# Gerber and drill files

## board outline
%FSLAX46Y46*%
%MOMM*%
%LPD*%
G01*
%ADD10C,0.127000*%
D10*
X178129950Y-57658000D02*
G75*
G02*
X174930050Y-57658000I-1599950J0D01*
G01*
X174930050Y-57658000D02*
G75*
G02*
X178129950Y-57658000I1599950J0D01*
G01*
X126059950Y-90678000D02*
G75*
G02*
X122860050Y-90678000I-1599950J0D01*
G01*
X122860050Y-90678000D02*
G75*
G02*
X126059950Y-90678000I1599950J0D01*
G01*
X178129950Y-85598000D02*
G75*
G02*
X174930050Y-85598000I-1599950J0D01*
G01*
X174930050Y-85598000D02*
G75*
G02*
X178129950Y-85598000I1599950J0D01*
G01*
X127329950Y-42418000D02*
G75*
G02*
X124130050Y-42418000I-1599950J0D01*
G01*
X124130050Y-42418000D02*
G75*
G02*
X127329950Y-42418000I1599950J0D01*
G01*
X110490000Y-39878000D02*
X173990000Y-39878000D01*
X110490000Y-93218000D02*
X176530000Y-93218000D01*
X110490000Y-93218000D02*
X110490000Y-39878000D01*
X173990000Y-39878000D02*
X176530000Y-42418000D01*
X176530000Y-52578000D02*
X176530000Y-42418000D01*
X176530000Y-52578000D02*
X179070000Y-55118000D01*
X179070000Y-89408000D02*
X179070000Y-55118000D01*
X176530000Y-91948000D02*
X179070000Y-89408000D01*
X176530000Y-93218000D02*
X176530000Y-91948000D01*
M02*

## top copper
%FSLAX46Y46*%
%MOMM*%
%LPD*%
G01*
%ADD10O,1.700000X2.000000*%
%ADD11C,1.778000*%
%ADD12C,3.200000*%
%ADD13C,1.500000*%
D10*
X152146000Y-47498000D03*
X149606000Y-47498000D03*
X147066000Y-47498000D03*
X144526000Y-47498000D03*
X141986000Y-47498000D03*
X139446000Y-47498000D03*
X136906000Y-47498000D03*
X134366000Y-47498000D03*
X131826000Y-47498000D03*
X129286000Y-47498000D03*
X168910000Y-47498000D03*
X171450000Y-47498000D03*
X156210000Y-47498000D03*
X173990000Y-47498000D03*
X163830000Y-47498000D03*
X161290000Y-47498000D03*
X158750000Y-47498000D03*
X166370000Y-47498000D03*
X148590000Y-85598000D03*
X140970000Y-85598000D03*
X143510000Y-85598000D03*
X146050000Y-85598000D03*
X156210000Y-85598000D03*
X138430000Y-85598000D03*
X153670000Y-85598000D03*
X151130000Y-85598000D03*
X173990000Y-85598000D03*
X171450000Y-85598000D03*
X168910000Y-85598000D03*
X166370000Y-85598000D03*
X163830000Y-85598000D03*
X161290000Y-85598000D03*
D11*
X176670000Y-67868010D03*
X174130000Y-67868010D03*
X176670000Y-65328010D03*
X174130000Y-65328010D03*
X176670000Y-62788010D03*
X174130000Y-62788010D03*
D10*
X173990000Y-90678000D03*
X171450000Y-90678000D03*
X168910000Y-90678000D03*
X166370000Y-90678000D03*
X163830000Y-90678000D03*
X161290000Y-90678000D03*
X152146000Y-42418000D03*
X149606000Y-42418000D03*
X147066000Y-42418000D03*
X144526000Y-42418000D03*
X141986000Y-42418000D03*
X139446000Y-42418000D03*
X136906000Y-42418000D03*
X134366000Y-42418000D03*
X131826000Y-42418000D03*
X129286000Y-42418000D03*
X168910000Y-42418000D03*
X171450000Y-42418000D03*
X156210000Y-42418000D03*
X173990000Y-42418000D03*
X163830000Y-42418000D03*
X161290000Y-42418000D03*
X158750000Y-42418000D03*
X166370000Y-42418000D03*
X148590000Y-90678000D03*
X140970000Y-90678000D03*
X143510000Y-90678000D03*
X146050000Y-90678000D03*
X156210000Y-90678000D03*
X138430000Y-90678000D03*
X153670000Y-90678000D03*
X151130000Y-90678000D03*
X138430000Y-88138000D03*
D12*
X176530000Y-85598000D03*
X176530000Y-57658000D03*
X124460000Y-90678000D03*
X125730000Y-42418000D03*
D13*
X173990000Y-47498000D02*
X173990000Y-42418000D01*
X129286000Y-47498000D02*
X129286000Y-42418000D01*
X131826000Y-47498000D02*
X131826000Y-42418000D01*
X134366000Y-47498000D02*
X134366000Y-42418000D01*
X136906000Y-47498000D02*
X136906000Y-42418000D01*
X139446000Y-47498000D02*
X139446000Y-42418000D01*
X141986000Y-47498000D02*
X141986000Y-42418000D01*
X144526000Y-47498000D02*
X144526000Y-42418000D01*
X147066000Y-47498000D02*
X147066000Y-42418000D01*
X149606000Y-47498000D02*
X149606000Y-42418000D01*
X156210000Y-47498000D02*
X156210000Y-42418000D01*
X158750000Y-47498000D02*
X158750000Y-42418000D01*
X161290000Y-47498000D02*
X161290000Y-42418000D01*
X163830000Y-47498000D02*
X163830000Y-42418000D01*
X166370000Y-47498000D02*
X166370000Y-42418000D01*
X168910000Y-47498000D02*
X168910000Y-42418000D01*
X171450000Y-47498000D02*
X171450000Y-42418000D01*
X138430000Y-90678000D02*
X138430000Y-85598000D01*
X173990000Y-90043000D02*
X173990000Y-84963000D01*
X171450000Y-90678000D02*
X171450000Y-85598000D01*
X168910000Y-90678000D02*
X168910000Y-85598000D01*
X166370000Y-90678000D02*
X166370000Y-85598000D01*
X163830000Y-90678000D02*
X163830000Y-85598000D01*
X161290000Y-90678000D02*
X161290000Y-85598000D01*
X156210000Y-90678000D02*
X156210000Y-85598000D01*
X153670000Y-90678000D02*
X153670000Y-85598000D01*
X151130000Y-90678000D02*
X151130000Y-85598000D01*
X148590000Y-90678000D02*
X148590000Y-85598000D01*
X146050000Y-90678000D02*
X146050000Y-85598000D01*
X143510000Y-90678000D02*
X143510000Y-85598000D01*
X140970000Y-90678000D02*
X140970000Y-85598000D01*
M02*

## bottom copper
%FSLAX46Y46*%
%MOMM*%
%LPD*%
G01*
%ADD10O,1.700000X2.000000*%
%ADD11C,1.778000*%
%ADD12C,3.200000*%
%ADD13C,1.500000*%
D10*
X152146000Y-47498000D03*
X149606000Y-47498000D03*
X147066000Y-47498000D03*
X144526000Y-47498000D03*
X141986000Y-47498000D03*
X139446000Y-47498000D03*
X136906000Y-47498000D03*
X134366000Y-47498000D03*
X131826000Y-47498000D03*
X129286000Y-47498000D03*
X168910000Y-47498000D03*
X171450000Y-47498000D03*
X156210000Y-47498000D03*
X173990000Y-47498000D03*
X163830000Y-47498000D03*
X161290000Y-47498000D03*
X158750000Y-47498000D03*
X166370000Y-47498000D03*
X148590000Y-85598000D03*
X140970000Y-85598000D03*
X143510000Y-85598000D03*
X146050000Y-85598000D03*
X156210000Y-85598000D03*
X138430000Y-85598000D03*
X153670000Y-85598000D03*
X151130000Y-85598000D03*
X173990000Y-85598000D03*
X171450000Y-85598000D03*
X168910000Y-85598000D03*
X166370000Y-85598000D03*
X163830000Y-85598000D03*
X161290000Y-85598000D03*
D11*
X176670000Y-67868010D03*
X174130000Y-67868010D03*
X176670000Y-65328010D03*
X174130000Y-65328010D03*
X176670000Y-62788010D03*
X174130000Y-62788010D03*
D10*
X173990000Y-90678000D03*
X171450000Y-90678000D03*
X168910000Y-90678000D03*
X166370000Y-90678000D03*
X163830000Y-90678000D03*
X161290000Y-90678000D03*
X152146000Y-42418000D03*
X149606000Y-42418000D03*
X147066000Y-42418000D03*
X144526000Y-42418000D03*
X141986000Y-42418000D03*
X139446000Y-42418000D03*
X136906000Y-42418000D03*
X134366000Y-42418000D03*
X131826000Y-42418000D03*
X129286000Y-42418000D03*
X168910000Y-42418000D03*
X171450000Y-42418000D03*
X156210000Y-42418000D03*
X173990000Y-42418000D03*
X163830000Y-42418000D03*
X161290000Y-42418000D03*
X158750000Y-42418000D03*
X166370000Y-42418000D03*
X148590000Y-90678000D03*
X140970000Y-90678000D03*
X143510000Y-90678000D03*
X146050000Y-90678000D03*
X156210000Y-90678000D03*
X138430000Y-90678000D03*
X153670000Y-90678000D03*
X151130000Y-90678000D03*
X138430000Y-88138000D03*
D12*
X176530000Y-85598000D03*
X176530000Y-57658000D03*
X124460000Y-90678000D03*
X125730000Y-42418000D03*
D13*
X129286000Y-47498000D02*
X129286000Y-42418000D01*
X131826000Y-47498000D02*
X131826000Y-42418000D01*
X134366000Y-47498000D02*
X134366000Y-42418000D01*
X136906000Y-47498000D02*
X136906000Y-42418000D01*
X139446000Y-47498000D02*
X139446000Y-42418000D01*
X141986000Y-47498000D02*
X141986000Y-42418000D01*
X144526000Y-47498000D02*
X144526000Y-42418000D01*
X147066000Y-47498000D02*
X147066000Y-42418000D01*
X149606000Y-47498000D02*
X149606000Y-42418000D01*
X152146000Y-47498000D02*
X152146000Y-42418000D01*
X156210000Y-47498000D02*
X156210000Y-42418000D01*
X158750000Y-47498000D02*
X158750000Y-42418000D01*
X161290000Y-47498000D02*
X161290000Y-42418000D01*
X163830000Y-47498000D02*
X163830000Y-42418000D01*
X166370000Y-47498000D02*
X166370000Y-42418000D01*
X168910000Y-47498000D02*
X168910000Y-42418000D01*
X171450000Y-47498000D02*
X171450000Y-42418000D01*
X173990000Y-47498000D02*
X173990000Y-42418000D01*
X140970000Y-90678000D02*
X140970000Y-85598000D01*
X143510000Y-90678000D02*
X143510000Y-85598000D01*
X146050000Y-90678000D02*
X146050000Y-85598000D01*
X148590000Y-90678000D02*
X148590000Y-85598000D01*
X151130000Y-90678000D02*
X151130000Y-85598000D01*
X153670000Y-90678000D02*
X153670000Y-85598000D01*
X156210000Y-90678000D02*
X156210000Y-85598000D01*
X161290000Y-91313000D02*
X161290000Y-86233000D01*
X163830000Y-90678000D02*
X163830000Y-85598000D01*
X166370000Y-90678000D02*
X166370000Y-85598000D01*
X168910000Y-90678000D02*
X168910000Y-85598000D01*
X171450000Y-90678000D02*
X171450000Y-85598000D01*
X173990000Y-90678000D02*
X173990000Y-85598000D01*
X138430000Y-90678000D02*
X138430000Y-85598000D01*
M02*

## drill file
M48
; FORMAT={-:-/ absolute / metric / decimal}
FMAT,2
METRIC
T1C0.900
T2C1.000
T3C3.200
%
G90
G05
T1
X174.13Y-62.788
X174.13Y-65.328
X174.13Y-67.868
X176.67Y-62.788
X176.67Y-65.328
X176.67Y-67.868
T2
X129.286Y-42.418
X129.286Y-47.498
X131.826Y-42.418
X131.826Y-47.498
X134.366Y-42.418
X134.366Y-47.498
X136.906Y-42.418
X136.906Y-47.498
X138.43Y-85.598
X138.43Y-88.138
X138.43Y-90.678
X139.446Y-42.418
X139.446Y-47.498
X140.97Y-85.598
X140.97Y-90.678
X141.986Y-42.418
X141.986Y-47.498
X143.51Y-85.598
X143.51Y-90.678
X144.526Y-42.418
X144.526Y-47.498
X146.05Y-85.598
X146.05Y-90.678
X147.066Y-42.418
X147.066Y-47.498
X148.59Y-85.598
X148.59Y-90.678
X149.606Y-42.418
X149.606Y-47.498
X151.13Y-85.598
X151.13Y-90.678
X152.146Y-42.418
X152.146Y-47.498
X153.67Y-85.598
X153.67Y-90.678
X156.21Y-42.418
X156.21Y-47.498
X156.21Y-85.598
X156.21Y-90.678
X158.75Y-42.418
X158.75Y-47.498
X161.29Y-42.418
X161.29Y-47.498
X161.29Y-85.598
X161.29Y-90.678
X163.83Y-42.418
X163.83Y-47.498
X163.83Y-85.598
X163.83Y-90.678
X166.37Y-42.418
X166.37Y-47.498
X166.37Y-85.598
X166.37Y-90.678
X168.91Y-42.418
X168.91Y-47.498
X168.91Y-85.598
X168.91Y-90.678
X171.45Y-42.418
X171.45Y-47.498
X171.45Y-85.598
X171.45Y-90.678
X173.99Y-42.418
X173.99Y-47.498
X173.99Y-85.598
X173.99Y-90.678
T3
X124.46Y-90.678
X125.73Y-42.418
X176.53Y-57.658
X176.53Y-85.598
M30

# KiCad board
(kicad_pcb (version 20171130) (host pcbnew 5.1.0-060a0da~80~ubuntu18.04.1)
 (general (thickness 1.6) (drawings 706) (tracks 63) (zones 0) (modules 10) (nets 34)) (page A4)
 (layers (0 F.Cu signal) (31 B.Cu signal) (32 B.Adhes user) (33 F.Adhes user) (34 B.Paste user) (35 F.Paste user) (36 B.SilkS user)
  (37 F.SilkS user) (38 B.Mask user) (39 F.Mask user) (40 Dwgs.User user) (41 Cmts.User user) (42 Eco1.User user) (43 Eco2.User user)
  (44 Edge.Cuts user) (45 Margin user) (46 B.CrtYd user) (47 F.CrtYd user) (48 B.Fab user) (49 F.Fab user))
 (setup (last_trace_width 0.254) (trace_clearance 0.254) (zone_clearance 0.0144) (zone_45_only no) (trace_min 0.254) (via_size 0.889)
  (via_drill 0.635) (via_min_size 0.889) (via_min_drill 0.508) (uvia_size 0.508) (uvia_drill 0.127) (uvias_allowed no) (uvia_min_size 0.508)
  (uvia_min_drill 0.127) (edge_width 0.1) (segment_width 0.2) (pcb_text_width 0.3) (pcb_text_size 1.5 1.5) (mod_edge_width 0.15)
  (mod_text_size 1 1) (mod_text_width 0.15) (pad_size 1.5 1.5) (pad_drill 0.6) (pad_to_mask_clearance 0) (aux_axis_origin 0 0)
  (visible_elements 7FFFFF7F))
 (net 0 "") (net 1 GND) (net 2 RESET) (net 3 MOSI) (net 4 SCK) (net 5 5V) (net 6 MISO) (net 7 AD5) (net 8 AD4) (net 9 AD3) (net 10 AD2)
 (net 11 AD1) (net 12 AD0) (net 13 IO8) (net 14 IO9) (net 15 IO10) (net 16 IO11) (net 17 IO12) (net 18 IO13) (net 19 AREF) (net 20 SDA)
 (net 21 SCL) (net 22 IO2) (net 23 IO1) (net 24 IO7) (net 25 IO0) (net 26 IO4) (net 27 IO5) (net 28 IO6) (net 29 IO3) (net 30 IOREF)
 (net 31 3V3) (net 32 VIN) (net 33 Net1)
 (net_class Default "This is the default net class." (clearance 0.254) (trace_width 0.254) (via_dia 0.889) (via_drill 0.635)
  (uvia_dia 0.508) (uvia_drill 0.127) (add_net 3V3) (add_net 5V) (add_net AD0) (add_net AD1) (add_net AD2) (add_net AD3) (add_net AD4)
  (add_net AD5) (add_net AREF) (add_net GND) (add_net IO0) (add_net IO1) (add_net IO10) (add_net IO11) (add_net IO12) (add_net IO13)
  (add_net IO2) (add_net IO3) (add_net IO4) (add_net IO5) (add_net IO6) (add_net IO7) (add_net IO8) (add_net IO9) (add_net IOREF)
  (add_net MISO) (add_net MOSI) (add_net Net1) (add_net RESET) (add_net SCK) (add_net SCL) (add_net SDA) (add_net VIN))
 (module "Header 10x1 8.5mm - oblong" (layer F.Cu) (at 152.146 47.498)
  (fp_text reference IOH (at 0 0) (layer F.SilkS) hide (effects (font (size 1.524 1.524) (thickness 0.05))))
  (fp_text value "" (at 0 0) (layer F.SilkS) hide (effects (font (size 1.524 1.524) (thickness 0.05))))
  (pad 1 thru_hole oval (at 0 0 180) (size 1.7 2) (drill 1) (layers *.Cu *.Paste *.Mask))
  (pad 2 thru_hole oval (at -2.54 0 180) (size 1.7 2) (drill 1) (layers *.Cu *.Paste *.Mask))
  (pad 3 thru_hole oval (at -5.08 0 180) (size 1.7 2) (drill 1) (layers *.Cu *.Paste *.Mask))
  (pad 4 thru_hole oval (at -7.62 0 180) (size 1.7 2) (drill 1) (layers *.Cu *.Paste *.Mask))
  (pad 5 thru_hole oval (at -10.16 0 180) (size 1.7 2) (drill 1) (layers *.Cu *.Paste *.Mask))
  (pad 6 thru_hole oval (at -12.7 0 180) (size 1.7 2) (drill 1) (layers *.Cu *.Paste *.Mask))
  (pad 7 thru_hole oval (at -15.24 0 180) (size 1.7 2) (drill 1) (layers *.Cu *.Paste *.Mask))
  (pad 8 thru_hole oval (at -17.78 0 180) (size 1.7 2) (drill 1) (layers *.Cu *.Paste *.Mask))
  (pad 9 thru_hole oval (at -20.32 0 180) (size 1.7 2) (drill 1) (layers *.Cu *.Paste *.Mask))
  (pad 10 thru_hole oval (at -22.86 0 180) (size 1.7 2) (drill 1) (layers *.Cu *.Paste *.Mask)))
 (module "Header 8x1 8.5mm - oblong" (layer F.Cu) (at 173.99 47.498)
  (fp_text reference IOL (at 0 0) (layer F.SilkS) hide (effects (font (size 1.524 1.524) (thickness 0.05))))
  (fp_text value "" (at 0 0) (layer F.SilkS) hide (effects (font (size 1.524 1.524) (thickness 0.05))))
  (pad 3 thru_hole oval (at -5.08 0 180) (size 1.7 2) (drill 1) (layers *.Cu *.Paste *.Mask))
  (pad 2 thru_hole oval (at -2.54 0 180) (size 1.7 2) (drill 1) (layers *.Cu *.Paste *.Mask))
  (pad 8 thru_hole oval (at -17.78 0 180) (size 1.7 2) (drill 1) (layers *.Cu *.Paste *.Mask))
  (pad 1 thru_hole oval (at 0 0 180) (size 1.7 2) (drill 1) (layers *.Cu *.Paste *.Mask))
  (pad 5 thru_hole oval (at -10.16 0 180) (size 1.7 2) (drill 1) (layers *.Cu *.Paste *.Mask))
  (pad 6 thru_hole oval (at -12.7 0 180) (size 1.7 2) (drill 1) (layers *.Cu *.Paste *.Mask))
  (pad 7 thru_hole oval (at -15.24 0 180) (size 1.7 2) (drill 1) (layers *.Cu *.Paste *.Mask))
  (pad 4 thru_hole oval (at -7.62 0 180) (size 1.7 2) (drill 1) (layers *.Cu *.Paste *.Mask)))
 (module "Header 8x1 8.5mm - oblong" (layer F.Cu) (at 156.21 85.598)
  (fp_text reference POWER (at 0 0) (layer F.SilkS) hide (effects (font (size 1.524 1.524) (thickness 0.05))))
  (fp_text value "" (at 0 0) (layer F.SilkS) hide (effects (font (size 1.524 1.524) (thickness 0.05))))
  (pad 4 thru_hole oval (at -7.62 0 180) (size 1.7 2) (drill 1) (layers *.Cu *.Paste *.Mask))
  (pad 7 thru_hole oval (at -15.24 0 180) (size 1.7 2) (drill 1) (layers *.Cu *.Paste *.Mask))
  (pad 6 thru_hole oval (at -12.7 0 180) (size 1.7 2) (drill 1) (layers *.Cu *.Paste *.Mask))
  (pad 5 thru_hole oval (at -10.16 0 180) (size 1.7 2) (drill 1) (layers *.Cu *.Paste *.Mask))
  (pad 1 thru_hole oval (at 0 0 180) (size 1.7 2) (drill 1) (layers *.Cu *.Paste *.Mask))
  (pad 8 thru_hole oval (at -17.78 0 180) (size 1.7 2) (drill 1) (layers *.Cu *.Paste *.Mask))
  (pad 2 thru_hole oval (at -2.54 0 180) (size 1.7 2) (drill 1) (layers *.Cu *.Paste *.Mask))
  (pad 3 thru_hole oval (at -5.08 0 180) (size 1.7 2) (drill 1) (layers *.Cu *.Paste *.Mask)))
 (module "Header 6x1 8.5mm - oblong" (layer F.Cu) (at 161.29 85.598)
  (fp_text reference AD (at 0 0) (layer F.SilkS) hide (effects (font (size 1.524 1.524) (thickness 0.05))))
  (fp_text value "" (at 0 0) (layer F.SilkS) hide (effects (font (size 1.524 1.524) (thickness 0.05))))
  (pad 6 thru_hole oval (at 12.7 0) (size 1.7 2) (drill 1) (layers *.Cu *.Paste *.Mask))
  (pad 5 thru_hole oval (at 10.16 0) (size 1.7 2) (drill 1) (layers *.Cu *.Paste *.Mask))
  (pad 4 thru_hole oval (at 7.62 0) (size 1.7 2) (drill 1) (layers *.Cu *.Paste *.Mask))
  (pad 3 thru_hole oval (at 5.08 0) (size 1.7 2) (drill 1) (layers *.Cu *.Paste *.Mask))
  (pad 2 thru_hole oval (at 2.54 0) (size 1.7 2) (drill 1) (layers *.Cu *.Paste *.Mask))
  (pad 1 thru_hole oval (at 0 0) (size 1.7 2) (drill 1) (layers *.Cu *.Paste *.Mask)))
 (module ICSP (layer F.Cu) (at 174.13 62.78801)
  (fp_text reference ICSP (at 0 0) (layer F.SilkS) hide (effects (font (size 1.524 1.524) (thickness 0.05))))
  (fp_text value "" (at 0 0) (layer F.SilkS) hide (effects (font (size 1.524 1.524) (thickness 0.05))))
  (pad 6 thru_hole circle (at 2.54 5.08) (size 1.778 1.778) (drill 0.9) (layers *.Cu *.Paste *.Mask) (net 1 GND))
  (pad 5 thru_hole circle (at 0 5.08) (size 1.778 1.778) (drill 0.9) (layers *.Cu *.Paste *.Mask) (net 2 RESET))
  (pad 4 thru_hole circle (at 2.54 2.54) (size 1.778 1.778) (drill 0.9) (layers *.Cu *.Paste *.Mask) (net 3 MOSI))
  (pad 3 thru_hole circle (at 0 2.54) (size 1.778 1.778) (drill 0.9) (layers *.Cu *.Paste *.Mask) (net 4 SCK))
  (pad 2 thru_hole circle (at 2.54 0) (size 1.778 1.778) (drill 0.9) (layers *.Cu *.Paste *.Mask) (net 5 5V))
  (pad 1 thru_hole circle (at 0 0) (size 1.778 1.778) (drill 0.9) (layers *.Cu *.Paste *.Mask) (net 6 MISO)))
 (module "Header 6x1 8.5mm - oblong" (layer F.Cu) (at 161.29 90.678)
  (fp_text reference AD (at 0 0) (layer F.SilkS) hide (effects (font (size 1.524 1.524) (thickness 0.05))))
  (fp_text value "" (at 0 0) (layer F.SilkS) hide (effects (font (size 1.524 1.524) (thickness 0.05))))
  (pad 6 thru_hole oval (at 12.7 0) (size 1.7 2) (drill 1) (layers *.Cu *.Paste *.Mask) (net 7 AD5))
  (pad 5 thru_hole oval (at 10.16 0) (size 1.7 2) (drill 1) (layers *.Cu *.Paste *.Mask) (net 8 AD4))
  (pad 4 thru_hole oval (at 7.62 0) (size 1.7 2) (drill 1) (layers *.Cu *.Paste *.Mask) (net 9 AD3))
  (pad 3 thru_hole oval (at 5.08 0) (size 1.7 2) (drill 1) (layers *.Cu *.Paste *.Mask) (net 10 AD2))
  (pad 2 thru_hole oval (at 2.54 0) (size 1.7 2) (drill 1) (layers *.Cu *.Paste *.Mask) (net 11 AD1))
  (pad 1 thru_hole oval (at 0 0) (size 1.7 2) (drill 1) (layers *.Cu *.Paste *.Mask) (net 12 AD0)))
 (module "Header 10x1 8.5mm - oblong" (layer F.Cu) (at 152.146 42.418)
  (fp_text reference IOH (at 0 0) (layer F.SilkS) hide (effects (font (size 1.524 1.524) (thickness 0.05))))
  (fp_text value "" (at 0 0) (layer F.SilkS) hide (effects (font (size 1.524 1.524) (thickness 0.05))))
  (pad 1 thru_hole oval (at 0 0 180) (size 1.7 2) (drill 1) (layers *.Cu *.Paste *.Mask) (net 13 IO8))
  (pad 2 thru_hole oval (at -2.54 0 180) (size 1.7 2) (drill 1) (layers *.Cu *.Paste *.Mask) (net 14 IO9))
  (pad 3 thru_hole oval (at -5.08 0 180) (size 1.7 2) (drill 1) (layers *.Cu *.Paste *.Mask) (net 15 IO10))
  (pad 4 thru_hole oval (at -7.62 0 180) (size 1.7 2) (drill 1) (layers *.Cu *.Paste *.Mask) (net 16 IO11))
  (pad 5 thru_hole oval (at -10.16 0 180) (size 1.7 2) (drill 1) (layers *.Cu *.Paste *.Mask) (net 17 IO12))
  (pad 6 thru_hole oval (at -12.7 0 180) (size 1.7 2) (drill 1) (layers *.Cu *.Paste *.Mask) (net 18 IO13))
  (pad 7 thru_hole oval (at -15.24 0 180) (size 1.7 2) (drill 1) (layers *.Cu *.Paste *.Mask) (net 1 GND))
  (pad 8 thru_hole oval (at -17.78 0 180) (size 1.7 2) (drill 1) (layers *.Cu *.Paste *.Mask) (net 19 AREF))
  (pad 9 thru_hole oval (at -20.32 0 180) (size 1.7 2) (drill 1) (layers *.Cu *.Paste *.Mask) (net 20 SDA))
  (pad 10 thru_hole oval (at -22.86 0 180) (size 1.7 2) (drill 1) (layers *.Cu *.Paste *.Mask) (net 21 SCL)))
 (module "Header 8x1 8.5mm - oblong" (layer F.Cu) (at 173.99 42.418)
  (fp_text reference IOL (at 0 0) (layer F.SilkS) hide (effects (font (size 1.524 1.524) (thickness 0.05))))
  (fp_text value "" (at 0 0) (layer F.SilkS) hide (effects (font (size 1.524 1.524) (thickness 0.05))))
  (pad 3 thru_hole oval (at -5.08 0 180) (size 1.7 2) (drill 1) (layers *.Cu *.Paste *.Mask) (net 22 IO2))
  (pad 2 thru_hole oval (at -2.54 0 180) (size 1.7 2) (drill 1) (layers *.Cu *.Paste *.Mask) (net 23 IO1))
  (pad 8 thru_hole oval (at -17.78 0 180) (size 1.7 2) (drill 1) (layers *.Cu *.Paste *.Mask) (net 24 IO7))
  (pad 1 thru_hole oval (at 0 0 180) (size 1.7 2) (drill 1) (layers *.Cu *.Paste *.Mask) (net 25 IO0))
  (pad 5 thru_hole oval (at -10.16 0 180) (size 1.7 2) (drill 1) (layers *.Cu *.Paste *.Mask) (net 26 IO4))
  (pad 6 thru_hole oval (at -12.7 0 180) (size 1.7 2) (drill 1) (layers *.Cu *.Paste *.Mask) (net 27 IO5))
  (pad 7 thru_hole oval (at -15.24 0 180) (size 1.7 2) (drill 1) (layers *.Cu *.Paste *.Mask) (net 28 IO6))
  (pad 4 thru_hole oval (at -7.62 0 180) (size 1.7 2) (drill 1) (layers *.Cu *.Paste *.Mask) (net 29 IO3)))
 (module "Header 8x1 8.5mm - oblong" (layer F.Cu) (at 156.21 90.678)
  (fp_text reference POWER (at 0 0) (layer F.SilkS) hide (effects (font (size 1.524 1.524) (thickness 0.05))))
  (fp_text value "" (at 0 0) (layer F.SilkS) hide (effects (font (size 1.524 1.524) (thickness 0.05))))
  (pad 4 thru_hole oval (at -7.62 0 180) (size 1.7 2) (drill 1) (layers *.Cu *.Paste *.Mask) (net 5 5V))
  (pad 7 thru_hole oval (at -15.24 0 180) (size 1.7 2) (drill 1) (layers *.Cu *.Paste *.Mask) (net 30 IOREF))
  (pad 6 thru_hole oval (at -12.7 0 180) (size 1.7 2) (drill 1) (layers *.Cu *.Paste *.Mask) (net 2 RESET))
  (pad 5 thru_hole oval (at -10.16 0 180) (size 1.7 2) (drill 1) (layers *.Cu *.Paste *.Mask) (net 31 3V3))
  (pad 1 thru_hole oval (at 0 0 180) (size 1.7 2) (drill 1) (layers *.Cu *.Paste *.Mask) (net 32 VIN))
  (pad 8 thru_hole oval (at -17.78 0 180) (size 1.7 2) (drill 1) (layers *.Cu *.Paste *.Mask))
  (pad 2 thru_hole oval (at -2.54 0 180) (size 1.7 2) (drill 1) (layers *.Cu *.Paste *.Mask) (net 1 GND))
  (pad 3 thru_hole oval (at -5.08 0 180) (size 1.7 2) (drill 1) (layers *.Cu *.Paste *.Mask) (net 1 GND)))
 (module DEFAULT (layer F.Cu) (at 80.01 124.46)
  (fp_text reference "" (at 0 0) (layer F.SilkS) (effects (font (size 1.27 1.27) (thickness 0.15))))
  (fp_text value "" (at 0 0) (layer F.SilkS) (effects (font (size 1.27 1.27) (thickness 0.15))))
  (pad 1 thru_hole oval (at 58.42 -36.322) (size 1.7 2) (drill 1) (layers *.Cu *.Paste *.Mask))
  (pad 0 thru_hole circle (at 96.52 -38.862) (size 3.2 3.2) (drill 3.2) (layers *.Cu *.Paste *.Mask))
  (pad 0 thru_hole circle (at 96.52 -66.802) (size 3.2 3.2) (drill 3.2) (layers *.Cu *.Paste *.Mask))
  (pad 0 thru_hole circle (at 44.45 -33.782) (size 3.2 3.2) (drill 3.2) (layers *.Cu *.Paste *.Mask))
  (pad 0 thru_hole circle (at 45.72 -82.042) (size 3.2 3.2) (drill 3.2) (layers *.Cu *.Paste *.Mask)))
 (gr_arc (start 176.53 57.658) (end 178.12995 57.658) (angle -360) (layer Edge.Cuts) (width 0.127))
 (gr_arc (start 124.46 90.678) (end 126.05995 90.678) (angle -360) (layer Edge.Cuts) (width 0.127))
 (gr_arc (start 176.53 85.598) (end 178.12995 85.598) (angle -360) (layer Edge.Cuts) (width 0.127))
 (gr_arc (start 125.73 42.418) (end 127.32995 42.418) (angle -360) (layer Edge.Cuts) (width 0.127))
 (gr_line (start 110.49 39.878) (end 173.99 39.878) (layer Edge.Cuts) (width 0.127))
 (gr_line (start 110.49 93.218) (end 176.53 93.218) (layer Edge.Cuts) (width 0.127))
 (gr_line (start 110.49 93.218) (end 110.49 39.878) (layer Edge.Cuts) (width 0.127))
 (gr_line (start 173.99 39.878) (end 176.53 42.418) (layer Edge.Cuts) (width 0.127))
 (gr_line (start 176.53 52.578) (end 176.53 42.418) (layer Edge.Cuts) (width 0.127))
 (gr_line (start 176.53 52.578) (end 179.07 55.118) (layer Edge.Cuts) (width 0.127))
 (gr_line (start 179.07 89.408) (end 179.07 55.118) (layer Edge.Cuts) (width 0.127))
 (gr_line (start 176.53 91.948) (end 179.07 89.408) (layer Edge.Cuts) (width 0.127))
 (gr_line (start 176.53 93.218) (end 176.53 91.948) (layer Edge.Cuts) (width 0.127))
 (segment (start 173.99 47.498) (end 173.99 42.418) (width 1.5) (layer F.Cu) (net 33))
 (segment (start 129.286 47.498) (end 129.286 42.418) (width 1.5) (layer F.Cu) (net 33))
 (segment (start 131.826 47.498) (end 131.826 42.418) (width 1.5) (layer F.Cu) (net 33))
 (segment (start 134.366 47.498) (end 134.366 42.418) (width 1.5) (layer F.Cu) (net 33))
 (segment (start 136.906 47.498) (end 136.906 42.418) (width 1.5) (layer F.Cu) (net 33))
 (segment (start 139.446 47.498) (end 139.446 42.418) (width 1.5) (layer F.Cu) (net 33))
 (segment (start 141.986 47.498) (end 141.986 42.418) (width 1.5) (layer F.Cu) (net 33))
 (segment (start 144.526 47.498) (end 144.526 42.418) (width 1.5) (layer F.Cu) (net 33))
 (segment (start 147.066 47.498) (end 147.066 42.418) (width 1.5) (layer F.Cu) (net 33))
 (segment (start 149.606 47.498) (end 149.606 42.418) (width 1.5) (layer F.Cu) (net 33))
 (segment (start 156.21 47.498) (end 156.21 42.418) (width 1.5) (layer F.Cu) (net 33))
 (segment (start 158.75 47.498) (end 158.75 42.418) (width 1.5) (layer F.Cu) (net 33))
 (segment (start 161.29 47.498) (end 161.29 42.418) (width 1.5) (layer F.Cu) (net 33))
 (segment (start 163.83 47.498) (end 163.83 42.418) (width 1.5) (layer F.Cu) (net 33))
 (segment (start 166.37 47.498) (end 166.37 42.418) (width 1.5) (layer F.Cu) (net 33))
 (segment (start 168.91 47.498) (end 168.91 42.418) (width 1.5) (layer F.Cu) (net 33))
 (segment (start 171.45 47.498) (end 171.45 42.418) (width 1.5) (layer F.Cu) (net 33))
 (segment (start 138.43 90.678) (end 138.43 85.598) (width 1.5) (layer F.Cu) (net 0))
 (segment (start 173.99 90.043) (end 173.99 84.963) (width 1.5) (layer F.Cu) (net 33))
 (segment (start 171.45 90.678) (end 171.45 85.598) (width 1.5) (layer F.Cu) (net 33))
 (segment (start 168.91 90.678) (end 168.91 85.598) (width 1.5) (layer F.Cu) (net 33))
 (segment (start 166.37 90.678) (end 166.37 85.598) (width 1.5) (layer F.Cu) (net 33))
 (segment (start 163.83 90.678) (end 163.83 85.598) (width 1.5) (layer F.Cu) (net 33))
 (segment (start 161.29 90.678) (end 161.29 85.598) (width 1.5) (layer F.Cu) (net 33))
 (segment (start 156.21 90.678) (end 156.21 85.598) (width 1.5) (layer F.Cu) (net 33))
 (segment (start 153.67 90.678) (end 153.67 85.598) (width 1.5) (layer F.Cu) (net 33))
 (segment (start 151.13 90.678) (end 151.13 85.598) (width 1.5) (layer F.Cu) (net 33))
 (segment (start 148.59 90.678) (end 148.59 85.598) (width 1.5) (layer F.Cu) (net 33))
 (segment (start 146.05 90.678) (end 146.05 85.598) (width 1.5) (layer F.Cu) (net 33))
 (segment (start 143.51 90.678) (end 143.51 85.598) (width 1.5) (layer F.Cu) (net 33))
 (segment (start 140.97 90.678) (end 140.97 85.598) (width 1.5) (layer F.Cu) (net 33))
 (segment (start 129.286 47.498) (end 129.286 42.418) (width 1.5) (layer B.Cu) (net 33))
 (segment (start 131.826 47.498) (end 131.826 42.418) (width 1.5) (layer B.Cu) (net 33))
 (segment (start 134.366 47.498) (end 134.366 42.418) (width 1.5) (layer B.Cu) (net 33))
 (segment (start 136.906 47.498) (end 136.906 42.418) (width 1.5) (layer B.Cu) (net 33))
 (segment (start 139.446 47.498) (end 139.446 42.418) (width 1.5) (layer B.Cu) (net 33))
 (segment (start 141.986 47.498) (end 141.986 42.418) (width 1.5) (layer B.Cu) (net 33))
 (segment (start 144.526 47.498) (end 144.526 42.418) (width 1.5) (layer B.Cu) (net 33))
 (segment (start 147.066 47.498) (end 147.066 42.418) (width 1.5) (layer B.Cu) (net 33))
 (segment (start 149.606 47.498) (end 149.606 42.418) (width 1.5) (layer B.Cu) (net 33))
 (segment (start 152.146 47.498) (end 152.146 42.418) (width 1.5) (layer B.Cu) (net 33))
 (segment (start 156.21 47.498) (end 156.21 42.418) (width 1.5) (layer B.Cu) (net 33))
 (segment (start 158.75 47.498) (end 158.75 42.418) (width 1.5) (layer B.Cu) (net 33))
 (segment (start 161.29 47.498) (end 161.29 42.418) (width 1.5) (layer B.Cu) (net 33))
 (segment (start 163.83 47.498) (end 163.83 42.418) (width 1.5) (layer B.Cu) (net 33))
 (segment (start 166.37 47.498) (end 166.37 42.418) (width 1.5) (layer B.Cu) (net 33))
 (segment (start 168.91 47.498) (end 168.91 42.418) (width 1.5) (layer B.Cu) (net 33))
 (segment (start 171.45 47.498) (end 171.45 42.418) (width 1.5) (layer B.Cu) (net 33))
 (segment (start 173.99 47.498) (end 173.99 42.418) (width 1.5) (layer B.Cu) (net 33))
 (segment (start 140.97 90.678) (end 140.97 85.598) (width 1.5) (layer B.Cu) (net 33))
 (segment (start 143.51 90.678) (end 143.51 85.598) (width 1.5) (layer B.Cu) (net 33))
 (segment (start 146.05 90.678) (end 146.05 85.598) (width 1.5) (layer B.Cu) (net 33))
 (segment (start 148.59 90.678) (end 148.59 85.598) (width 1.5) (layer B.Cu) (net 33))
 (segment (start 151.13 90.678) (end 151.13 85.598) (width 1.5) (layer B.Cu) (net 33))
 (segment (start 153.67 90.678) (end 153.67 85.598) (width 1.5) (layer B.Cu) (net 33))
 (segment (start 156.21 90.678) (end 156.21 85.598) (width 1.5) (layer B.Cu) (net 33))
 (segment (start 161.29 91.313) (end 161.29 86.233) (width 1.5) (layer B.Cu) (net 33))
 (segment (start 163.83 90.678) (end 163.83 85.598) (width 1.5) (layer B.Cu) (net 33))
 (segment (start 166.37 90.678) (end 166.37 85.598) (width 1.5) (layer B.Cu) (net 33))
 (segment (start 168.91 90.678) (end 168.91 85.598) (width 1.5) (layer B.Cu) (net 33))
 (segment (start 171.45 90.678) (end 171.45 85.598) (width 1.5) (layer B.Cu) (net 33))
 (segment (start 173.99 90.678) (end 173.99 85.598) (width 1.5) (layer B.Cu) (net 33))
 (segment (start 138.43 90.678) (end 138.43 85.598) (width 1.5) (layer B.Cu) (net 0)))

